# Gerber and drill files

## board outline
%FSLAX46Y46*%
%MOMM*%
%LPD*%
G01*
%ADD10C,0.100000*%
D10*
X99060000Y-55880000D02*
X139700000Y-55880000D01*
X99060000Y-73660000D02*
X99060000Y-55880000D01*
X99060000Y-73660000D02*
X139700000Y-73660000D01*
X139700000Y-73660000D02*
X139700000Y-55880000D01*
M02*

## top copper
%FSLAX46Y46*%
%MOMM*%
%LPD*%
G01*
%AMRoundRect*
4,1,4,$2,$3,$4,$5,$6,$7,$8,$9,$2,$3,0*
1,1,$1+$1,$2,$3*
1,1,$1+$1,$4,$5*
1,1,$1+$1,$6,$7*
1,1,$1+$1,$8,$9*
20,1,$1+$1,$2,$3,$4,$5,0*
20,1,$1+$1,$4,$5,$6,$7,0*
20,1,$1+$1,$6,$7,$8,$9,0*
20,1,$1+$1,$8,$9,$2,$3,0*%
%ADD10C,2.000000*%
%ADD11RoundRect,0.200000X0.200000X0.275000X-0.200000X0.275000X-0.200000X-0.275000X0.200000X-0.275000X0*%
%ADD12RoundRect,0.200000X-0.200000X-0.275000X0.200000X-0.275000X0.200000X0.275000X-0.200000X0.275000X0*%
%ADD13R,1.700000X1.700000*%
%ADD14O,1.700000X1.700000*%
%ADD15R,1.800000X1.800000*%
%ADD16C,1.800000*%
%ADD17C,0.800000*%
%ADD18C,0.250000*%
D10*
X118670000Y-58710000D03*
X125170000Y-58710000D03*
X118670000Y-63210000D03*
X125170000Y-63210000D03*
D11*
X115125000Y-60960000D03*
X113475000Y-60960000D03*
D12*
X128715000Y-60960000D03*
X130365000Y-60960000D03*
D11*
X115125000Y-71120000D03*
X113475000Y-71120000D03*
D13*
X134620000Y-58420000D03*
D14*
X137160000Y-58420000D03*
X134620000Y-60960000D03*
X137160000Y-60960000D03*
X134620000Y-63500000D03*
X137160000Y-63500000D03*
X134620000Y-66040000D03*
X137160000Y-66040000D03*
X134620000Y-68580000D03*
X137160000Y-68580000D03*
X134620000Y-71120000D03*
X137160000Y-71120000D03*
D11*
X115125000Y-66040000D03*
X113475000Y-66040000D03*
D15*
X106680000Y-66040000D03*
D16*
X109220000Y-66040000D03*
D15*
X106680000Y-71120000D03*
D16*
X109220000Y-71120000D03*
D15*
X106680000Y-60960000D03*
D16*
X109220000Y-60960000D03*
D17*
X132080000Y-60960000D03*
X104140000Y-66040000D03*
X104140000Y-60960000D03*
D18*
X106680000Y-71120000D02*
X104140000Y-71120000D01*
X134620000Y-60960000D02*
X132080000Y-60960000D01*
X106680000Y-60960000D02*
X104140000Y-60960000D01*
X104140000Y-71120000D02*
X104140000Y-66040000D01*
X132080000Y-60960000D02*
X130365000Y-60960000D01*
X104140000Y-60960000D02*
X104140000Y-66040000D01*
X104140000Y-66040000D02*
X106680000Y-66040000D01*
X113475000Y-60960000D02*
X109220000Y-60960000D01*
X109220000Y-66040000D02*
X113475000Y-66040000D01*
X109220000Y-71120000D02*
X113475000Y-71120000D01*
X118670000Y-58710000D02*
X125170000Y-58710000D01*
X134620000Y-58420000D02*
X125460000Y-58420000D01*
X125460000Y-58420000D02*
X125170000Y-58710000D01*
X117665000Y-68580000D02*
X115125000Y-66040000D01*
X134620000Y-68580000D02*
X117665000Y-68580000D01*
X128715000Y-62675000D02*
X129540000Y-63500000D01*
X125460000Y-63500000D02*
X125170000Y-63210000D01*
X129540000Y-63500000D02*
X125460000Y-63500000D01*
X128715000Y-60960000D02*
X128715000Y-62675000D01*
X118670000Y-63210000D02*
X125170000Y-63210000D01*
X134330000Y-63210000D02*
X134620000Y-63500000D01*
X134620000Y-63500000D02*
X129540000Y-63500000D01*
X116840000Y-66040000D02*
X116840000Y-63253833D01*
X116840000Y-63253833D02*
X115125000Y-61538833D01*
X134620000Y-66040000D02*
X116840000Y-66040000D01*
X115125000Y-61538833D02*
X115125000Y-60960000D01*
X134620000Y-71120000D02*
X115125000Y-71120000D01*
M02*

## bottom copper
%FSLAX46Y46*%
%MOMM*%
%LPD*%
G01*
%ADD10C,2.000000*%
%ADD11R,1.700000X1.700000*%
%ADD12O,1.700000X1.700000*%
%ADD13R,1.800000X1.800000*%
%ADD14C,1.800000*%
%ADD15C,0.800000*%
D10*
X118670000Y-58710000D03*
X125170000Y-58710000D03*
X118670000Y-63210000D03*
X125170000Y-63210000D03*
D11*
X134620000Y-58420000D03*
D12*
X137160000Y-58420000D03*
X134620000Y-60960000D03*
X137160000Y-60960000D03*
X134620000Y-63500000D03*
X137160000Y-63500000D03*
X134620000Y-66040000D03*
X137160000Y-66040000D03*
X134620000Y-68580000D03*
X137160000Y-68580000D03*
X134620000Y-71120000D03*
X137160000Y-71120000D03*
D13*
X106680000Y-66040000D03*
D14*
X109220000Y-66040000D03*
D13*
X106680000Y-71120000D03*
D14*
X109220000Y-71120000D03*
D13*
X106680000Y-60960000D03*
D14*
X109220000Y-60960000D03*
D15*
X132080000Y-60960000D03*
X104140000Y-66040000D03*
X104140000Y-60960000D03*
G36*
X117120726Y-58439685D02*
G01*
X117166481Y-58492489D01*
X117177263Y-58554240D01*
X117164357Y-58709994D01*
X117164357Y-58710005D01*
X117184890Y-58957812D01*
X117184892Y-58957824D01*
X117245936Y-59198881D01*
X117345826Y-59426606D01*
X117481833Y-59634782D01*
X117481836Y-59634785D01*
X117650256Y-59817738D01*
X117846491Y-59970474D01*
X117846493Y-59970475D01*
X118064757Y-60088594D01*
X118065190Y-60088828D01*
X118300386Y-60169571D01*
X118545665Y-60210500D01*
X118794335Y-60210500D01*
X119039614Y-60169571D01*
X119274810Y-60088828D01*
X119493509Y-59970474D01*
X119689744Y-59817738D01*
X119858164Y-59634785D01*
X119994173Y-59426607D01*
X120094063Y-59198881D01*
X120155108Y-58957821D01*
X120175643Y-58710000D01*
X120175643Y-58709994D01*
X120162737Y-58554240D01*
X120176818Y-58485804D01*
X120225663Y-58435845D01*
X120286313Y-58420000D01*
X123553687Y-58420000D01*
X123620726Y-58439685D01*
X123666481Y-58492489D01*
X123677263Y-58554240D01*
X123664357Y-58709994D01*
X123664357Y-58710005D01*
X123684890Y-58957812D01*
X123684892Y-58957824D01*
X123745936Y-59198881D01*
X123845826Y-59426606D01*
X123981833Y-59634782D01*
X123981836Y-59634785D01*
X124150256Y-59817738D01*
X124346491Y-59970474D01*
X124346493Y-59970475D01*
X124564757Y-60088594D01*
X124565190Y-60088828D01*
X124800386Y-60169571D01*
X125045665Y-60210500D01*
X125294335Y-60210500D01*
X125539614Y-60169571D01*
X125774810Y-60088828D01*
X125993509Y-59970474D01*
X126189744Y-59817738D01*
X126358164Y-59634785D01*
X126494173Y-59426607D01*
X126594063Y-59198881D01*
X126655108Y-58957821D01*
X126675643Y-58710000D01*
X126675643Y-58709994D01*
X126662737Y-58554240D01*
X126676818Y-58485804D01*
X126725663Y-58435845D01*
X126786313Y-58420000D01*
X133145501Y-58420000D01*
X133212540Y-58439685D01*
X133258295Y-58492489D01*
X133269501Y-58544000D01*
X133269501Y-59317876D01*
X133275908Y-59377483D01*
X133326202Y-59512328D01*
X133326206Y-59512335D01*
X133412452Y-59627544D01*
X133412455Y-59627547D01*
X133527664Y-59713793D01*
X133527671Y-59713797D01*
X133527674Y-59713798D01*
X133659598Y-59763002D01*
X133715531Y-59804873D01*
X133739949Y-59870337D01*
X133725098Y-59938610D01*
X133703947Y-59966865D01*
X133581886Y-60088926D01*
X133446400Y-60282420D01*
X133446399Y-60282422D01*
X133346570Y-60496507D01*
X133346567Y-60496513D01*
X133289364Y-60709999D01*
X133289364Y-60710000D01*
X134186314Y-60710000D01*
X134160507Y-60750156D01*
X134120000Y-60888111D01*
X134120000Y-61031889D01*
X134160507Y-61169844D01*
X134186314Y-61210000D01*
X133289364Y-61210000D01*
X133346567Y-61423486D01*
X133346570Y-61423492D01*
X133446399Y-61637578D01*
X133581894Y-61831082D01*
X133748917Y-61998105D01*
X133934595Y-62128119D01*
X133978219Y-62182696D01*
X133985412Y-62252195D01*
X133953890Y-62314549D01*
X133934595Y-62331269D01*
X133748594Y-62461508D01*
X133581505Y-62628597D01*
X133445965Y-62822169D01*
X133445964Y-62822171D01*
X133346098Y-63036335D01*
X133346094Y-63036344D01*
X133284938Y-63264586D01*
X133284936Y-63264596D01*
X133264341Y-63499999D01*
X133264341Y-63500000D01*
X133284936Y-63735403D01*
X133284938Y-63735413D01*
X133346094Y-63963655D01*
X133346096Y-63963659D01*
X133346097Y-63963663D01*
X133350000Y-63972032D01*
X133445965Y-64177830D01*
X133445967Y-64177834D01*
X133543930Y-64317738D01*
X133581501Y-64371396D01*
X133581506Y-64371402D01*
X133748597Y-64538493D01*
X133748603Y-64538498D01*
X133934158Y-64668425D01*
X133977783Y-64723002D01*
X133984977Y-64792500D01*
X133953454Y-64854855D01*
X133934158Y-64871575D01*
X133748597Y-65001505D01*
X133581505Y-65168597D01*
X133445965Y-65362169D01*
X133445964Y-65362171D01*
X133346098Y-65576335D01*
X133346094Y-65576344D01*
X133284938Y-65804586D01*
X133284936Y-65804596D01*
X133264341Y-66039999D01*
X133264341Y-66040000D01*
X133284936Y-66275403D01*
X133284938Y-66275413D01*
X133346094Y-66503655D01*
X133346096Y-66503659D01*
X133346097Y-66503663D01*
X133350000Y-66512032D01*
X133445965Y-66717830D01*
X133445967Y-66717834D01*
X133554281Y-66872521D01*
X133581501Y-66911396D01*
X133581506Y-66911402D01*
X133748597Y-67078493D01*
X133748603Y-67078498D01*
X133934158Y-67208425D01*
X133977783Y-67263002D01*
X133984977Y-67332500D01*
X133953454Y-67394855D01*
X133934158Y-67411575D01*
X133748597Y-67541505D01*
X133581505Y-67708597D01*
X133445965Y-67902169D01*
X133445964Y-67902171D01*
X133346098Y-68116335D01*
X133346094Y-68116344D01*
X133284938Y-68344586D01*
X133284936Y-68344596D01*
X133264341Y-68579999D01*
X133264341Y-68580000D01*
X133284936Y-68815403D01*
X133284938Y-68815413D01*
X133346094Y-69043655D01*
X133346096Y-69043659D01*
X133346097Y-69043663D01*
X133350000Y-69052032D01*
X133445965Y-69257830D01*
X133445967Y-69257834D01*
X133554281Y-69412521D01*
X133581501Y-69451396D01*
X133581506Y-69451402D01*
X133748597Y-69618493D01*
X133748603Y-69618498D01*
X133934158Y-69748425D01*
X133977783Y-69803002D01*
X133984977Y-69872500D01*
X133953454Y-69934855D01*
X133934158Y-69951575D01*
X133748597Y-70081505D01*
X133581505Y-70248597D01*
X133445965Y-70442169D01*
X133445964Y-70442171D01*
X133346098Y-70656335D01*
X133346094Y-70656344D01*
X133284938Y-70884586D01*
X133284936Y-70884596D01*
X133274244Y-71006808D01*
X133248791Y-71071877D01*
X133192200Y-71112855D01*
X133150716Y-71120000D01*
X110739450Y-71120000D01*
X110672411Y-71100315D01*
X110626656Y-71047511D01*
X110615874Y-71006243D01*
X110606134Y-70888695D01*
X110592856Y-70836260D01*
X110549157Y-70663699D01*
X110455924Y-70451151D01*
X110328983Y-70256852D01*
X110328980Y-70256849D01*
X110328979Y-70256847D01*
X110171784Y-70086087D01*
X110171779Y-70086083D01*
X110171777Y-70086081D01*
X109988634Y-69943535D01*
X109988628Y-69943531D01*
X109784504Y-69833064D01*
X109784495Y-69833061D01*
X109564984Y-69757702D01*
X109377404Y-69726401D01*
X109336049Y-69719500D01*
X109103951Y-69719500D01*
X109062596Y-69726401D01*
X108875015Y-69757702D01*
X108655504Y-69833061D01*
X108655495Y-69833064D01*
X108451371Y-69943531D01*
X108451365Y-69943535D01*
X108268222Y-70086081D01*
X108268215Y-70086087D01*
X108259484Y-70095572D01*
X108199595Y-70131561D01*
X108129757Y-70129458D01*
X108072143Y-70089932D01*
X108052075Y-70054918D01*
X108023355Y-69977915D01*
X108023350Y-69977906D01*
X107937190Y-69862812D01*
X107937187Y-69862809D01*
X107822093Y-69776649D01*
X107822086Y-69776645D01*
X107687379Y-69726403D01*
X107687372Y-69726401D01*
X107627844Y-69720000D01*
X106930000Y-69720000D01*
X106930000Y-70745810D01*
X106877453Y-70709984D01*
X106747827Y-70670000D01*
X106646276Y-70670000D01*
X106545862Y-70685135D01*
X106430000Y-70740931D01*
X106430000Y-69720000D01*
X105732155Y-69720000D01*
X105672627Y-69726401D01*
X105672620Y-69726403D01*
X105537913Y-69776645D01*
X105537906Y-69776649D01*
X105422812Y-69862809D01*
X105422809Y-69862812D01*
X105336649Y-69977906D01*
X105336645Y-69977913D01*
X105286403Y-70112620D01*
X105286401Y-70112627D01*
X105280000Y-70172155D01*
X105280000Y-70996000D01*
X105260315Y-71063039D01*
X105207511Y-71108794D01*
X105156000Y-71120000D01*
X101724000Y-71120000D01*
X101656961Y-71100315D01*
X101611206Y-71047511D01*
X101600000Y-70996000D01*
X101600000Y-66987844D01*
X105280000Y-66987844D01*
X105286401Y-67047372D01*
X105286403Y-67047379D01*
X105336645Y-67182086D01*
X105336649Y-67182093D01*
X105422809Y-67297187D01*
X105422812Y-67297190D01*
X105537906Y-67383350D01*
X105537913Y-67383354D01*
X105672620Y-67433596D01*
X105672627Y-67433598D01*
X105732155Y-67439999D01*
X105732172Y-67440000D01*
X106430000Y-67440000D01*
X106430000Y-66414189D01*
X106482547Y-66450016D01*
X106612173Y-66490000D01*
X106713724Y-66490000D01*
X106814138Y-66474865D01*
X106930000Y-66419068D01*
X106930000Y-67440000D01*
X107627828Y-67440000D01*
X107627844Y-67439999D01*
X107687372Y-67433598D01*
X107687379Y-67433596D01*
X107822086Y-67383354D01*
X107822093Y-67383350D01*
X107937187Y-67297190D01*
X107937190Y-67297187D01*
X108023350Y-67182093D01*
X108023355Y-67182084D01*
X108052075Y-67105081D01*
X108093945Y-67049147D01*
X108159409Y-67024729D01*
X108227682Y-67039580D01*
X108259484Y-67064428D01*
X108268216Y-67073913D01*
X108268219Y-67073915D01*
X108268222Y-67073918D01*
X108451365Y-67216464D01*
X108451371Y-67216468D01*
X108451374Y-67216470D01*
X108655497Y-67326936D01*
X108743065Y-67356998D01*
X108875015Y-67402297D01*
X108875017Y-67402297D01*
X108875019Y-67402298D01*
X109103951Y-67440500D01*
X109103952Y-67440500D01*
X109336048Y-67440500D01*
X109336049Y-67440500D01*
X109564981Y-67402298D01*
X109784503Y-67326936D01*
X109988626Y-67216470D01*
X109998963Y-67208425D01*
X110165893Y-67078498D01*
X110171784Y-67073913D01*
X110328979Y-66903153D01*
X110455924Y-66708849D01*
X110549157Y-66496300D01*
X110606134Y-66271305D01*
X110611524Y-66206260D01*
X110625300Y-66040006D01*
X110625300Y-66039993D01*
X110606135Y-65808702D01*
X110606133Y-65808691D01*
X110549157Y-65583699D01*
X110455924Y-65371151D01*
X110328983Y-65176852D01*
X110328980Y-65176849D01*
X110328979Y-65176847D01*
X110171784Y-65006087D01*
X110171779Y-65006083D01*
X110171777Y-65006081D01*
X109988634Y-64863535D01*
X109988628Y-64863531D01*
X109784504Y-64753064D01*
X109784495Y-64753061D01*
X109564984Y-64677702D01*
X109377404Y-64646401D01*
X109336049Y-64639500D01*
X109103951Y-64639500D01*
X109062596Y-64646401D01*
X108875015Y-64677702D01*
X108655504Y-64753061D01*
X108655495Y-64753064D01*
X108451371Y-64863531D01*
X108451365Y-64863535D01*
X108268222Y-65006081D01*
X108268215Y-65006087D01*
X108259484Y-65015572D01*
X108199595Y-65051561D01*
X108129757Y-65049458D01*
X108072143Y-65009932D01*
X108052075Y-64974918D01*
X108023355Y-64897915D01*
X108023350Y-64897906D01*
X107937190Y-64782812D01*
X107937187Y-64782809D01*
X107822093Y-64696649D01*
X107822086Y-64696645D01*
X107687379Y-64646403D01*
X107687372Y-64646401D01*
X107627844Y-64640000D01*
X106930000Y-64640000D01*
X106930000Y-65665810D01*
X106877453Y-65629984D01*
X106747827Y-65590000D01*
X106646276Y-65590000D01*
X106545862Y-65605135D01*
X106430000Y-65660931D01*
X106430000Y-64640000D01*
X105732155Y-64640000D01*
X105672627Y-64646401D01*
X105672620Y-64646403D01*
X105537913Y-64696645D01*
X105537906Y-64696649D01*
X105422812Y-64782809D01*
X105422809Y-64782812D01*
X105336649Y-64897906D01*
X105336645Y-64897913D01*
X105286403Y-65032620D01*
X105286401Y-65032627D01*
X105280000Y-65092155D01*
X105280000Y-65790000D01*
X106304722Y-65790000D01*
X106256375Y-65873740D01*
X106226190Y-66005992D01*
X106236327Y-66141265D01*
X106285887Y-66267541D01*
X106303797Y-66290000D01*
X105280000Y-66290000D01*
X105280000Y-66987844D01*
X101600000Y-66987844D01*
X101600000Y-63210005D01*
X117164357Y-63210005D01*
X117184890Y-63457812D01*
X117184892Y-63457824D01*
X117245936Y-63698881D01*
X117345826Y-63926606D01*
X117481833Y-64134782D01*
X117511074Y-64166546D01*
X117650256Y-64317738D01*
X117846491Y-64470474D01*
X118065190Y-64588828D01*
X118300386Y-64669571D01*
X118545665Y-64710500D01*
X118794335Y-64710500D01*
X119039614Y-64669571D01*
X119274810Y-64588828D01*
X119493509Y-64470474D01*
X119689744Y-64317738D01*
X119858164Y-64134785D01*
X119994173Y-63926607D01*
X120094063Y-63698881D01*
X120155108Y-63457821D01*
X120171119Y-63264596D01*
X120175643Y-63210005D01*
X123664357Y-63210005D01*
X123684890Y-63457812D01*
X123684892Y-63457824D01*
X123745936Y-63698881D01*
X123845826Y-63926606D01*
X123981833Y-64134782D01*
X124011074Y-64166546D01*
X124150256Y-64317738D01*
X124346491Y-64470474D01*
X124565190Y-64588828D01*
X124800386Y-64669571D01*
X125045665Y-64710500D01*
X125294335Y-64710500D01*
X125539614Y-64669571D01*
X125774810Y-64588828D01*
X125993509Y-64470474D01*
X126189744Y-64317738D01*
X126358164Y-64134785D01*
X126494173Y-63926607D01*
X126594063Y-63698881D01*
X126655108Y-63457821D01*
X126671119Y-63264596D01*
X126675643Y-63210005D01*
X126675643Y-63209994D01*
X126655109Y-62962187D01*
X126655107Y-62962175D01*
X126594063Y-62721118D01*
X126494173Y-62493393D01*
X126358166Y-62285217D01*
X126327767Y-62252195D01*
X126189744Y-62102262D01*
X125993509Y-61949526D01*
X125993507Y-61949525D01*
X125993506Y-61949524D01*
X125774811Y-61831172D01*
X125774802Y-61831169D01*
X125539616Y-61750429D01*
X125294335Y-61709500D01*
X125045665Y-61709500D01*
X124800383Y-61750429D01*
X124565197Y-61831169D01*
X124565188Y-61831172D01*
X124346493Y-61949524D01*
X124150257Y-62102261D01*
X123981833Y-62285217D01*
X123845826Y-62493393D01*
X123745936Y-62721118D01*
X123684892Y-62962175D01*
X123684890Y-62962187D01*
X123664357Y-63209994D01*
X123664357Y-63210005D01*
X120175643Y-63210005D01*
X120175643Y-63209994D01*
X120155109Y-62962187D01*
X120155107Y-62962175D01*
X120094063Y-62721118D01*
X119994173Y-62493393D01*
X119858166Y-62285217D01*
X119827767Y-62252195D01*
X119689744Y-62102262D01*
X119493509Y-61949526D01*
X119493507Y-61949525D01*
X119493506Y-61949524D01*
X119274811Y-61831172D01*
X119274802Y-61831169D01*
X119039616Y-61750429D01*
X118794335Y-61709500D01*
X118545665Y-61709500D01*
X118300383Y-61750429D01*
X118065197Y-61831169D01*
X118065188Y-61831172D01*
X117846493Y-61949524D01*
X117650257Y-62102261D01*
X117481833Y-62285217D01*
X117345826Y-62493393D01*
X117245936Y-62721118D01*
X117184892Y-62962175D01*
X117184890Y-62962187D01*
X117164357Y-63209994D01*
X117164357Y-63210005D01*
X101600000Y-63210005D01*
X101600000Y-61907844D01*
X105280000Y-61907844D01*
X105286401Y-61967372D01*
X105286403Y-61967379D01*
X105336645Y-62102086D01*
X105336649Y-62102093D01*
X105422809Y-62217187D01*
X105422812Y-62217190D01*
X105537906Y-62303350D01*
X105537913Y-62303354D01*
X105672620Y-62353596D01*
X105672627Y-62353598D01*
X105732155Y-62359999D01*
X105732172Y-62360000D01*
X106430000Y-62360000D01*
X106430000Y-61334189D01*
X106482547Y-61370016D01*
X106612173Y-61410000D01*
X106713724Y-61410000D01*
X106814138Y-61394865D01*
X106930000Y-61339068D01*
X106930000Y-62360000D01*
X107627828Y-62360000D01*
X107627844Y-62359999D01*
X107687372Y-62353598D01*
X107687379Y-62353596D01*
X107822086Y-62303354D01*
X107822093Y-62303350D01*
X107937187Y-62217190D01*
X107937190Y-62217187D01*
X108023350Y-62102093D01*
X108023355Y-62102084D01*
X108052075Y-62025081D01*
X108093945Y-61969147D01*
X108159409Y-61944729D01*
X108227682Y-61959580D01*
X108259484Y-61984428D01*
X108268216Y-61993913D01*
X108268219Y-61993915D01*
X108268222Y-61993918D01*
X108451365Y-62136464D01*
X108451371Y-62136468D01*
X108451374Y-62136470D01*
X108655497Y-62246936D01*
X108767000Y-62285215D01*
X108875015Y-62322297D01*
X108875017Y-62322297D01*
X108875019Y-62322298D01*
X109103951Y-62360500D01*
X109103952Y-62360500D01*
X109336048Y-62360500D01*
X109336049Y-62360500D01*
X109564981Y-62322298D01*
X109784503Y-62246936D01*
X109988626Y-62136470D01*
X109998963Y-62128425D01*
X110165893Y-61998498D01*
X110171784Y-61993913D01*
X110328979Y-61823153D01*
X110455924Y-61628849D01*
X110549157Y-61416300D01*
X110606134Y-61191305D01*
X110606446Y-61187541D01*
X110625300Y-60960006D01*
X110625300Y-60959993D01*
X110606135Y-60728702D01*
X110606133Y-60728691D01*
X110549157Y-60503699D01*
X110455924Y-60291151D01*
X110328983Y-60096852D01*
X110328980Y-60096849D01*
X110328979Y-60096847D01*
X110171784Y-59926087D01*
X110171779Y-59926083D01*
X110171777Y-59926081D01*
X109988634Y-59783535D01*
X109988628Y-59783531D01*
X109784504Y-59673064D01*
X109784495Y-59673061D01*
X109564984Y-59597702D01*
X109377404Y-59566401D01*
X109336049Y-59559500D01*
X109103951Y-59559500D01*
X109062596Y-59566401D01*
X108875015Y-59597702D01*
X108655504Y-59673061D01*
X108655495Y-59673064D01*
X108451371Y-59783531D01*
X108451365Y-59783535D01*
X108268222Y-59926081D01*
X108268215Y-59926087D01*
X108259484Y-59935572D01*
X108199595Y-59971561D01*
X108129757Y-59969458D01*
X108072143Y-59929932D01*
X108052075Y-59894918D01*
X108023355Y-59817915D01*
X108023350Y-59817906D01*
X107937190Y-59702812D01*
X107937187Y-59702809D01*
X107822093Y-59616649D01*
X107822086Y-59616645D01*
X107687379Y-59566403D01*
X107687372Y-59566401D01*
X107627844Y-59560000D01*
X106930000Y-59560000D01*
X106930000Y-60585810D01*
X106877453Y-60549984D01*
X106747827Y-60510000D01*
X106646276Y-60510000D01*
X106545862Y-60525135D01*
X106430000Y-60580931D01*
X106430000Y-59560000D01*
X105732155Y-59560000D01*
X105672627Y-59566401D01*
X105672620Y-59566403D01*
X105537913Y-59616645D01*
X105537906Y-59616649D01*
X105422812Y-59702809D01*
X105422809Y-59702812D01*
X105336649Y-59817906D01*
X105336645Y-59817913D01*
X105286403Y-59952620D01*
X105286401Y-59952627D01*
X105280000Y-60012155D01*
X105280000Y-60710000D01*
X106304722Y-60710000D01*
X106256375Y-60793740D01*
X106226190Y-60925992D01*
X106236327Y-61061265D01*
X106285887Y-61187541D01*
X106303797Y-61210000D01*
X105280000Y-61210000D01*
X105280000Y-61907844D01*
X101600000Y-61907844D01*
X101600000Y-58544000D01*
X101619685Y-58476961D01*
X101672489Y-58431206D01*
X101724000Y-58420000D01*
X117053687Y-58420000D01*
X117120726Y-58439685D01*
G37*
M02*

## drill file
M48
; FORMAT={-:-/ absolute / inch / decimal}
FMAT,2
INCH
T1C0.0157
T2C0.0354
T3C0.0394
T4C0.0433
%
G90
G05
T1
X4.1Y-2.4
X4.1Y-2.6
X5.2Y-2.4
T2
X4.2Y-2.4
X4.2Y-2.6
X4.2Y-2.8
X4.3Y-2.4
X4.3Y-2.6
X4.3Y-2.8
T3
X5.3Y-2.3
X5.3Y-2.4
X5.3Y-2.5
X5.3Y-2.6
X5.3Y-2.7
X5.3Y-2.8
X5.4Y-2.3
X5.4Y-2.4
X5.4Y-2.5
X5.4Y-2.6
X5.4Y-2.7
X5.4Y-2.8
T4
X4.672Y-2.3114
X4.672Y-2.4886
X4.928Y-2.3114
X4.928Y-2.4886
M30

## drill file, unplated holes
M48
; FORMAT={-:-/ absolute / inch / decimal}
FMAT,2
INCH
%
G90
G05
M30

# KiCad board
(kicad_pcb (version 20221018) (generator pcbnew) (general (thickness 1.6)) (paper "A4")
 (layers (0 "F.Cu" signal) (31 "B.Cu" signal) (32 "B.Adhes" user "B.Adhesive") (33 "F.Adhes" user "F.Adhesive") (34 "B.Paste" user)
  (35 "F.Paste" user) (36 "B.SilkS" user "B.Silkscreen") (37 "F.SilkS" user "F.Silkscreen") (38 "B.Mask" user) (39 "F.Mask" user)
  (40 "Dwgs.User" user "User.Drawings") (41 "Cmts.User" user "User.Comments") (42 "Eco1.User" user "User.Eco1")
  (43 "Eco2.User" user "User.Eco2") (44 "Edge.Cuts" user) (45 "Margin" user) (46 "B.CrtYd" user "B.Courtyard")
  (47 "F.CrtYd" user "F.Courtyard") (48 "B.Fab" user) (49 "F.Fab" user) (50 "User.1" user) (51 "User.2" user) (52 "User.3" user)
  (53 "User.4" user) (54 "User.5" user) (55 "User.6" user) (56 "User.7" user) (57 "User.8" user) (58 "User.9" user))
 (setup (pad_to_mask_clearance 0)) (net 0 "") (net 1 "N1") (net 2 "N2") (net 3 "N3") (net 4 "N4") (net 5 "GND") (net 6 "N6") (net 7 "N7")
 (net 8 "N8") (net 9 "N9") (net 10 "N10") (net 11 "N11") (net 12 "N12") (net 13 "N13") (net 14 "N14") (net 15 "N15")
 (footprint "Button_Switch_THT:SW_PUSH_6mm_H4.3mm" (layer "F.Cu") (at 118.67 58.71)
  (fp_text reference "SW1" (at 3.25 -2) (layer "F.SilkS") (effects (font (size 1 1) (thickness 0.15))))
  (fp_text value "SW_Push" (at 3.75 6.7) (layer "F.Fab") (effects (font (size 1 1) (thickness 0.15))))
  (pad "1" thru_hole circle (at 0 0 90) (size 2 2) (drill 1.1) (layers "*.Cu" "*.Mask") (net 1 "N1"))
  (pad "1" thru_hole circle (at 6.5 0 90) (size 2 2) (drill 1.1) (layers "*.Cu" "*.Mask") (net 1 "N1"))
  (pad "2" thru_hole circle (at 0 4.5 90) (size 2 2) (drill 1.1) (layers "*.Cu" "*.Mask") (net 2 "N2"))
  (pad "2" thru_hole circle (at 6.5 4.5 90) (size 2 2) (drill 1.1) (layers "*.Cu" "*.Mask") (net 2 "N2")))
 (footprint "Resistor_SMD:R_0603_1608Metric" (layer "F.Cu") (at 114.3 60.96 180)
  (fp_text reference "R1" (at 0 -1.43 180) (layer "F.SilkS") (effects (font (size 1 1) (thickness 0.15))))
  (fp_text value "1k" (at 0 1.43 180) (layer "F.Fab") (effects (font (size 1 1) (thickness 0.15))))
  (pad "1" smd roundrect (at -0.825 0 180) (size 0.8 0.95) (layers "F.Cu" "F.Paste" "F.Mask") (roundrect_rratio 0.25) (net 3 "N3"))
  (pad "2" smd roundrect (at 0.825 0 180) (size 0.8 0.95) (layers "F.Cu" "F.Paste" "F.Mask") (roundrect_rratio 0.25) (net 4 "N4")))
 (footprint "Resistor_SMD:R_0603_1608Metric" (layer "F.Cu") (at 129.54 60.96)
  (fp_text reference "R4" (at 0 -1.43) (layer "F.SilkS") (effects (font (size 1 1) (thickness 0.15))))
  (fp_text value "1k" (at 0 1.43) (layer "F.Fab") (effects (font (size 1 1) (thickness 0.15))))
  (pad "1" smd roundrect (at -0.825 0) (size 0.8 0.95) (layers "F.Cu" "F.Paste" "F.Mask") (roundrect_rratio 0.25) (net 2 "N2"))
  (pad "2" smd roundrect (at 0.825 0) (size 0.8 0.95) (layers "F.Cu" "F.Paste" "F.Mask") (roundrect_rratio 0.25) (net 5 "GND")))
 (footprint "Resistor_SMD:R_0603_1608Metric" (layer "F.Cu") (at 114.3 71.12 180)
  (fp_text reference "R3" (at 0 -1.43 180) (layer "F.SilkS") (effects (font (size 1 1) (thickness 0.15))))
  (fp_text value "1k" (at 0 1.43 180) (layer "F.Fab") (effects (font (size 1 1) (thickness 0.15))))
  (pad "1" smd roundrect (at -0.825 0 180) (size 0.8 0.95) (layers "F.Cu" "F.Paste" "F.Mask") (roundrect_rratio 0.25) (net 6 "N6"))
  (pad "2" smd roundrect (at 0.825 0 180) (size 0.8 0.95) (layers "F.Cu" "F.Paste" "F.Mask") (roundrect_rratio 0.25) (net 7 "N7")))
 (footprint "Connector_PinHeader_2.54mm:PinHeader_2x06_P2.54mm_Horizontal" (layer "F.Cu") (at 134.62 58.42)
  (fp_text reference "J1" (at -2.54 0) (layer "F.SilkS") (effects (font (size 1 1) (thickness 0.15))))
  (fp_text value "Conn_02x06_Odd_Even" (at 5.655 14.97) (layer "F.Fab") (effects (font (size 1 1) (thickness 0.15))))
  (pad "1" thru_hole rect (at 0 0) (size 1.7 1.7) (drill 1) (layers "*.Cu" "*.Mask") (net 1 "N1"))
  (pad "2" thru_hole oval (at 2.54 0) (size 1.7 1.7) (drill 1) (layers "*.Cu" "*.Mask") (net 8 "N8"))
  (pad "3" thru_hole oval (at 0 2.54) (size 1.7 1.7) (drill 1) (layers "*.Cu" "*.Mask") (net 5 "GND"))
  (pad "4" thru_hole oval (at 2.54 2.54) (size 1.7 1.7) (drill 1) (layers "*.Cu" "*.Mask") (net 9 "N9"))
  (pad "5" thru_hole oval (at 0 5.08) (size 1.7 1.7) (drill 1) (layers "*.Cu" "*.Mask") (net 2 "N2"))
  (pad "6" thru_hole oval (at 2.54 5.08) (size 1.7 1.7) (drill 1) (layers "*.Cu" "*.Mask") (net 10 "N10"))
  (pad "7" thru_hole oval (at 0 7.62) (size 1.7 1.7) (drill 1) (layers "*.Cu" "*.Mask") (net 3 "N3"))
  (pad "8" thru_hole oval (at 2.54 7.62) (size 1.7 1.7) (drill 1) (layers "*.Cu" "*.Mask") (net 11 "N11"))
  (pad "9" thru_hole oval (at 0 10.16) (size 1.7 1.7) (drill 1) (layers "*.Cu" "*.Mask") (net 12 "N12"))
  (pad "10" thru_hole oval (at 2.54 10.16) (size 1.7 1.7) (drill 1) (layers "*.Cu" "*.Mask") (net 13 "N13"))
  (pad "11" thru_hole oval (at 0 12.7) (size 1.7 1.7) (drill 1) (layers "*.Cu" "*.Mask") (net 6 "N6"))
  (pad "12" thru_hole oval (at 2.54 12.7) (size 1.7 1.7) (drill 1) (layers "*.Cu" "*.Mask") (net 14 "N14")))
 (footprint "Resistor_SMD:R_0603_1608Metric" (layer "F.Cu") (at 114.3 66.04 180)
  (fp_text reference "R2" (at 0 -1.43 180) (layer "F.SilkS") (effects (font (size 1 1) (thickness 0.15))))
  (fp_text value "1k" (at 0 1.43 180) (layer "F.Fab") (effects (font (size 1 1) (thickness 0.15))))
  (pad "1" smd roundrect (at -0.825 0 180) (size 0.8 0.95) (layers "F.Cu" "F.Paste" "F.Mask") (roundrect_rratio 0.25) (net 12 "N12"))
  (pad "2" smd roundrect (at 0.825 0 180) (size 0.8 0.95) (layers "F.Cu" "F.Paste" "F.Mask") (roundrect_rratio 0.25) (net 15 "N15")))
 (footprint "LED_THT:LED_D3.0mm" (layer "F.Cu") (at 106.68 66.04)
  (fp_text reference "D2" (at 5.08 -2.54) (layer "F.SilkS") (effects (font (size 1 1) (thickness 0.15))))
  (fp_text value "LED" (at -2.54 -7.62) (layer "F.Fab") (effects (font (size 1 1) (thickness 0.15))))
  (pad "1" thru_hole rect (at 0 0) (size 1.8 1.8) (drill 0.9) (layers "*.Cu" "*.Mask") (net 5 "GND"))
  (pad "2" thru_hole circle (at 2.54 0) (size 1.8 1.8) (drill 0.9) (layers "*.Cu" "*.Mask") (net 15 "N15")))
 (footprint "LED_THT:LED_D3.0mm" (layer "F.Cu") (at 106.68 71.12)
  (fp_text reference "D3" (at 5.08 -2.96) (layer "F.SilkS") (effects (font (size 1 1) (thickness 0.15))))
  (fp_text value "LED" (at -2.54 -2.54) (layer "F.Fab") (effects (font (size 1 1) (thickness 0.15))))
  (pad "1" thru_hole rect (at 0 0) (size 1.8 1.8) (drill 0.9) (layers "*.Cu" "*.Mask") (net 5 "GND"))
  (pad "2" thru_hole circle (at 2.54 0) (size 1.8 1.8) (drill 0.9) (layers "*.Cu" "*.Mask") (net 7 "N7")))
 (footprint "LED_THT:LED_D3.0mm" (layer "F.Cu") (at 106.68 60.96)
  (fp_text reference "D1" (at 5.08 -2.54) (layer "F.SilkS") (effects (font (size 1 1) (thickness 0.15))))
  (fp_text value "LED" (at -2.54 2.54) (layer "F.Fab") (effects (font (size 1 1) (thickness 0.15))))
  (pad "1" thru_hole rect (at 0 0) (size 1.8 1.8) (drill 0.9) (layers "*.Cu" "*.Mask") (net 5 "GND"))
  (pad "2" thru_hole circle (at 2.54 0) (size 1.8 1.8) (drill 0.9) (layers "*.Cu" "*.Mask") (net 4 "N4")))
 (gr_line (start 99.06 55.88) (end 139.7 55.88) (stroke (width 0.1) (type default)) (layer "Edge.Cuts"))
 (gr_line (start 99.06 73.66) (end 99.06 55.88) (stroke (width 0.1) (type default)) (layer "Edge.Cuts"))
 (gr_line (start 99.06 73.66) (end 139.7 73.66) (stroke (width 0.1) (type default)) (layer "Edge.Cuts"))
 (gr_line (start 139.7 73.66) (end 139.7 55.88) (stroke (width 0.1) (type default)) (layer "Edge.Cuts"))
 (segment (start 106.68 71.12) (end 104.14 71.12) (width 0.25) (layer "F.Cu") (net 5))
 (segment (start 134.62 60.96) (end 132.08 60.96) (width 0.25) (layer "F.Cu") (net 5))
 (segment (start 106.68 60.96) (end 104.14 60.96) (width 0.25) (layer "F.Cu") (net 5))
 (segment (start 104.14 71.12) (end 104.14 66.04) (width 0.25) (layer "F.Cu") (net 5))
 (segment (start 132.08 60.96) (end 130.365 60.96) (width 0.25) (layer "F.Cu") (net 5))
 (segment (start 104.14 60.96) (end 104.14 66.04) (width 0.25) (layer "F.Cu") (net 5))
 (segment (start 104.14 66.04) (end 106.68 66.04) (width 0.25) (layer "F.Cu") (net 5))
 (via (at 132.08 60.96) (size 0.8) (drill 0.4) (layers "F.Cu" "B.Cu") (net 5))
 (via (at 104.14 66.04) (size 0.8) (drill 0.4) (layers "F.Cu" "B.Cu") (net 5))
 (via (at 104.14 60.96) (size 0.8) (drill 0.4) (layers "F.Cu" "B.Cu") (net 5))
 (segment (start 113.475 60.96) (end 109.22 60.96) (width 0.25) (layer "F.Cu") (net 4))
 (segment (start 109.22 66.04) (end 113.475 66.04) (width 0.25) (layer "F.Cu") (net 15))
 (segment (start 109.22 71.12) (end 113.475 71.12) (width 0.25) (layer "F.Cu") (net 7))
 (segment (start 118.67 58.71) (end 125.17 58.71) (width 0.25) (layer "F.Cu") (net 1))
 (segment (start 134.62 58.42) (end 125.46 58.42) (width 0.25) (layer "F.Cu") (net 1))
 (segment (start 125.46 58.42) (end 125.17 58.71) (width 0.25) (layer "F.Cu") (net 1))
 (segment (start 117.665 68.58) (end 115.125 66.04) (width 0.25) (layer "F.Cu") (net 12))
 (segment (start 134.62 68.58) (end 117.665 68.58) (width 0.25) (layer "F.Cu") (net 12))
 (segment (start 128.715 62.675) (end 129.54 63.5) (width 0.25) (layer "F.Cu") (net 2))
 (segment (start 125.46 63.5) (end 125.17 63.21) (width 0.25) (layer "F.Cu") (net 2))
 (segment (start 129.54 63.5) (end 125.46 63.5) (width 0.25) (layer "F.Cu") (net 2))
 (segment (start 128.715 60.96) (end 128.715 62.675) (width 0.25) (layer "F.Cu") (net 2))
 (segment (start 118.67 63.21) (end 125.17 63.21) (width 0.25) (layer "F.Cu") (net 2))
 (segment (start 134.33 63.21) (end 134.62 63.5) (width 0.25) (layer "F.Cu") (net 2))
 (segment (start 134.62 63.5) (end 129.54 63.5) (width 0.25) (layer "F.Cu") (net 2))
 (segment (start 116.84 66.04) (end 116.84 63.253833) (width 0.25) (layer "F.Cu") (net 3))
 (segment (start 116.84 63.253833) (end 115.125 61.538833) (width 0.25) (layer "F.Cu") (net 3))
 (segment (start 134.62 66.04) (end 116.84 66.04) (width 0.25) (layer "F.Cu") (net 3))
 (segment (start 115.125 61.538833) (end 115.125 60.96) (width 0.25) (layer "F.Cu") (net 3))
 (segment (start 134.62 71.12) (end 115.125 71.12) (width 0.25) (layer "F.Cu") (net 6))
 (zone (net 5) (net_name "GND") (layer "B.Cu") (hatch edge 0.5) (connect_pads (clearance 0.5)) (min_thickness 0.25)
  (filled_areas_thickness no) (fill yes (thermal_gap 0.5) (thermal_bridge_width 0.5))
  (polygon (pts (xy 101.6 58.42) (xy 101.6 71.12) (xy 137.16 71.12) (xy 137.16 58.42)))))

